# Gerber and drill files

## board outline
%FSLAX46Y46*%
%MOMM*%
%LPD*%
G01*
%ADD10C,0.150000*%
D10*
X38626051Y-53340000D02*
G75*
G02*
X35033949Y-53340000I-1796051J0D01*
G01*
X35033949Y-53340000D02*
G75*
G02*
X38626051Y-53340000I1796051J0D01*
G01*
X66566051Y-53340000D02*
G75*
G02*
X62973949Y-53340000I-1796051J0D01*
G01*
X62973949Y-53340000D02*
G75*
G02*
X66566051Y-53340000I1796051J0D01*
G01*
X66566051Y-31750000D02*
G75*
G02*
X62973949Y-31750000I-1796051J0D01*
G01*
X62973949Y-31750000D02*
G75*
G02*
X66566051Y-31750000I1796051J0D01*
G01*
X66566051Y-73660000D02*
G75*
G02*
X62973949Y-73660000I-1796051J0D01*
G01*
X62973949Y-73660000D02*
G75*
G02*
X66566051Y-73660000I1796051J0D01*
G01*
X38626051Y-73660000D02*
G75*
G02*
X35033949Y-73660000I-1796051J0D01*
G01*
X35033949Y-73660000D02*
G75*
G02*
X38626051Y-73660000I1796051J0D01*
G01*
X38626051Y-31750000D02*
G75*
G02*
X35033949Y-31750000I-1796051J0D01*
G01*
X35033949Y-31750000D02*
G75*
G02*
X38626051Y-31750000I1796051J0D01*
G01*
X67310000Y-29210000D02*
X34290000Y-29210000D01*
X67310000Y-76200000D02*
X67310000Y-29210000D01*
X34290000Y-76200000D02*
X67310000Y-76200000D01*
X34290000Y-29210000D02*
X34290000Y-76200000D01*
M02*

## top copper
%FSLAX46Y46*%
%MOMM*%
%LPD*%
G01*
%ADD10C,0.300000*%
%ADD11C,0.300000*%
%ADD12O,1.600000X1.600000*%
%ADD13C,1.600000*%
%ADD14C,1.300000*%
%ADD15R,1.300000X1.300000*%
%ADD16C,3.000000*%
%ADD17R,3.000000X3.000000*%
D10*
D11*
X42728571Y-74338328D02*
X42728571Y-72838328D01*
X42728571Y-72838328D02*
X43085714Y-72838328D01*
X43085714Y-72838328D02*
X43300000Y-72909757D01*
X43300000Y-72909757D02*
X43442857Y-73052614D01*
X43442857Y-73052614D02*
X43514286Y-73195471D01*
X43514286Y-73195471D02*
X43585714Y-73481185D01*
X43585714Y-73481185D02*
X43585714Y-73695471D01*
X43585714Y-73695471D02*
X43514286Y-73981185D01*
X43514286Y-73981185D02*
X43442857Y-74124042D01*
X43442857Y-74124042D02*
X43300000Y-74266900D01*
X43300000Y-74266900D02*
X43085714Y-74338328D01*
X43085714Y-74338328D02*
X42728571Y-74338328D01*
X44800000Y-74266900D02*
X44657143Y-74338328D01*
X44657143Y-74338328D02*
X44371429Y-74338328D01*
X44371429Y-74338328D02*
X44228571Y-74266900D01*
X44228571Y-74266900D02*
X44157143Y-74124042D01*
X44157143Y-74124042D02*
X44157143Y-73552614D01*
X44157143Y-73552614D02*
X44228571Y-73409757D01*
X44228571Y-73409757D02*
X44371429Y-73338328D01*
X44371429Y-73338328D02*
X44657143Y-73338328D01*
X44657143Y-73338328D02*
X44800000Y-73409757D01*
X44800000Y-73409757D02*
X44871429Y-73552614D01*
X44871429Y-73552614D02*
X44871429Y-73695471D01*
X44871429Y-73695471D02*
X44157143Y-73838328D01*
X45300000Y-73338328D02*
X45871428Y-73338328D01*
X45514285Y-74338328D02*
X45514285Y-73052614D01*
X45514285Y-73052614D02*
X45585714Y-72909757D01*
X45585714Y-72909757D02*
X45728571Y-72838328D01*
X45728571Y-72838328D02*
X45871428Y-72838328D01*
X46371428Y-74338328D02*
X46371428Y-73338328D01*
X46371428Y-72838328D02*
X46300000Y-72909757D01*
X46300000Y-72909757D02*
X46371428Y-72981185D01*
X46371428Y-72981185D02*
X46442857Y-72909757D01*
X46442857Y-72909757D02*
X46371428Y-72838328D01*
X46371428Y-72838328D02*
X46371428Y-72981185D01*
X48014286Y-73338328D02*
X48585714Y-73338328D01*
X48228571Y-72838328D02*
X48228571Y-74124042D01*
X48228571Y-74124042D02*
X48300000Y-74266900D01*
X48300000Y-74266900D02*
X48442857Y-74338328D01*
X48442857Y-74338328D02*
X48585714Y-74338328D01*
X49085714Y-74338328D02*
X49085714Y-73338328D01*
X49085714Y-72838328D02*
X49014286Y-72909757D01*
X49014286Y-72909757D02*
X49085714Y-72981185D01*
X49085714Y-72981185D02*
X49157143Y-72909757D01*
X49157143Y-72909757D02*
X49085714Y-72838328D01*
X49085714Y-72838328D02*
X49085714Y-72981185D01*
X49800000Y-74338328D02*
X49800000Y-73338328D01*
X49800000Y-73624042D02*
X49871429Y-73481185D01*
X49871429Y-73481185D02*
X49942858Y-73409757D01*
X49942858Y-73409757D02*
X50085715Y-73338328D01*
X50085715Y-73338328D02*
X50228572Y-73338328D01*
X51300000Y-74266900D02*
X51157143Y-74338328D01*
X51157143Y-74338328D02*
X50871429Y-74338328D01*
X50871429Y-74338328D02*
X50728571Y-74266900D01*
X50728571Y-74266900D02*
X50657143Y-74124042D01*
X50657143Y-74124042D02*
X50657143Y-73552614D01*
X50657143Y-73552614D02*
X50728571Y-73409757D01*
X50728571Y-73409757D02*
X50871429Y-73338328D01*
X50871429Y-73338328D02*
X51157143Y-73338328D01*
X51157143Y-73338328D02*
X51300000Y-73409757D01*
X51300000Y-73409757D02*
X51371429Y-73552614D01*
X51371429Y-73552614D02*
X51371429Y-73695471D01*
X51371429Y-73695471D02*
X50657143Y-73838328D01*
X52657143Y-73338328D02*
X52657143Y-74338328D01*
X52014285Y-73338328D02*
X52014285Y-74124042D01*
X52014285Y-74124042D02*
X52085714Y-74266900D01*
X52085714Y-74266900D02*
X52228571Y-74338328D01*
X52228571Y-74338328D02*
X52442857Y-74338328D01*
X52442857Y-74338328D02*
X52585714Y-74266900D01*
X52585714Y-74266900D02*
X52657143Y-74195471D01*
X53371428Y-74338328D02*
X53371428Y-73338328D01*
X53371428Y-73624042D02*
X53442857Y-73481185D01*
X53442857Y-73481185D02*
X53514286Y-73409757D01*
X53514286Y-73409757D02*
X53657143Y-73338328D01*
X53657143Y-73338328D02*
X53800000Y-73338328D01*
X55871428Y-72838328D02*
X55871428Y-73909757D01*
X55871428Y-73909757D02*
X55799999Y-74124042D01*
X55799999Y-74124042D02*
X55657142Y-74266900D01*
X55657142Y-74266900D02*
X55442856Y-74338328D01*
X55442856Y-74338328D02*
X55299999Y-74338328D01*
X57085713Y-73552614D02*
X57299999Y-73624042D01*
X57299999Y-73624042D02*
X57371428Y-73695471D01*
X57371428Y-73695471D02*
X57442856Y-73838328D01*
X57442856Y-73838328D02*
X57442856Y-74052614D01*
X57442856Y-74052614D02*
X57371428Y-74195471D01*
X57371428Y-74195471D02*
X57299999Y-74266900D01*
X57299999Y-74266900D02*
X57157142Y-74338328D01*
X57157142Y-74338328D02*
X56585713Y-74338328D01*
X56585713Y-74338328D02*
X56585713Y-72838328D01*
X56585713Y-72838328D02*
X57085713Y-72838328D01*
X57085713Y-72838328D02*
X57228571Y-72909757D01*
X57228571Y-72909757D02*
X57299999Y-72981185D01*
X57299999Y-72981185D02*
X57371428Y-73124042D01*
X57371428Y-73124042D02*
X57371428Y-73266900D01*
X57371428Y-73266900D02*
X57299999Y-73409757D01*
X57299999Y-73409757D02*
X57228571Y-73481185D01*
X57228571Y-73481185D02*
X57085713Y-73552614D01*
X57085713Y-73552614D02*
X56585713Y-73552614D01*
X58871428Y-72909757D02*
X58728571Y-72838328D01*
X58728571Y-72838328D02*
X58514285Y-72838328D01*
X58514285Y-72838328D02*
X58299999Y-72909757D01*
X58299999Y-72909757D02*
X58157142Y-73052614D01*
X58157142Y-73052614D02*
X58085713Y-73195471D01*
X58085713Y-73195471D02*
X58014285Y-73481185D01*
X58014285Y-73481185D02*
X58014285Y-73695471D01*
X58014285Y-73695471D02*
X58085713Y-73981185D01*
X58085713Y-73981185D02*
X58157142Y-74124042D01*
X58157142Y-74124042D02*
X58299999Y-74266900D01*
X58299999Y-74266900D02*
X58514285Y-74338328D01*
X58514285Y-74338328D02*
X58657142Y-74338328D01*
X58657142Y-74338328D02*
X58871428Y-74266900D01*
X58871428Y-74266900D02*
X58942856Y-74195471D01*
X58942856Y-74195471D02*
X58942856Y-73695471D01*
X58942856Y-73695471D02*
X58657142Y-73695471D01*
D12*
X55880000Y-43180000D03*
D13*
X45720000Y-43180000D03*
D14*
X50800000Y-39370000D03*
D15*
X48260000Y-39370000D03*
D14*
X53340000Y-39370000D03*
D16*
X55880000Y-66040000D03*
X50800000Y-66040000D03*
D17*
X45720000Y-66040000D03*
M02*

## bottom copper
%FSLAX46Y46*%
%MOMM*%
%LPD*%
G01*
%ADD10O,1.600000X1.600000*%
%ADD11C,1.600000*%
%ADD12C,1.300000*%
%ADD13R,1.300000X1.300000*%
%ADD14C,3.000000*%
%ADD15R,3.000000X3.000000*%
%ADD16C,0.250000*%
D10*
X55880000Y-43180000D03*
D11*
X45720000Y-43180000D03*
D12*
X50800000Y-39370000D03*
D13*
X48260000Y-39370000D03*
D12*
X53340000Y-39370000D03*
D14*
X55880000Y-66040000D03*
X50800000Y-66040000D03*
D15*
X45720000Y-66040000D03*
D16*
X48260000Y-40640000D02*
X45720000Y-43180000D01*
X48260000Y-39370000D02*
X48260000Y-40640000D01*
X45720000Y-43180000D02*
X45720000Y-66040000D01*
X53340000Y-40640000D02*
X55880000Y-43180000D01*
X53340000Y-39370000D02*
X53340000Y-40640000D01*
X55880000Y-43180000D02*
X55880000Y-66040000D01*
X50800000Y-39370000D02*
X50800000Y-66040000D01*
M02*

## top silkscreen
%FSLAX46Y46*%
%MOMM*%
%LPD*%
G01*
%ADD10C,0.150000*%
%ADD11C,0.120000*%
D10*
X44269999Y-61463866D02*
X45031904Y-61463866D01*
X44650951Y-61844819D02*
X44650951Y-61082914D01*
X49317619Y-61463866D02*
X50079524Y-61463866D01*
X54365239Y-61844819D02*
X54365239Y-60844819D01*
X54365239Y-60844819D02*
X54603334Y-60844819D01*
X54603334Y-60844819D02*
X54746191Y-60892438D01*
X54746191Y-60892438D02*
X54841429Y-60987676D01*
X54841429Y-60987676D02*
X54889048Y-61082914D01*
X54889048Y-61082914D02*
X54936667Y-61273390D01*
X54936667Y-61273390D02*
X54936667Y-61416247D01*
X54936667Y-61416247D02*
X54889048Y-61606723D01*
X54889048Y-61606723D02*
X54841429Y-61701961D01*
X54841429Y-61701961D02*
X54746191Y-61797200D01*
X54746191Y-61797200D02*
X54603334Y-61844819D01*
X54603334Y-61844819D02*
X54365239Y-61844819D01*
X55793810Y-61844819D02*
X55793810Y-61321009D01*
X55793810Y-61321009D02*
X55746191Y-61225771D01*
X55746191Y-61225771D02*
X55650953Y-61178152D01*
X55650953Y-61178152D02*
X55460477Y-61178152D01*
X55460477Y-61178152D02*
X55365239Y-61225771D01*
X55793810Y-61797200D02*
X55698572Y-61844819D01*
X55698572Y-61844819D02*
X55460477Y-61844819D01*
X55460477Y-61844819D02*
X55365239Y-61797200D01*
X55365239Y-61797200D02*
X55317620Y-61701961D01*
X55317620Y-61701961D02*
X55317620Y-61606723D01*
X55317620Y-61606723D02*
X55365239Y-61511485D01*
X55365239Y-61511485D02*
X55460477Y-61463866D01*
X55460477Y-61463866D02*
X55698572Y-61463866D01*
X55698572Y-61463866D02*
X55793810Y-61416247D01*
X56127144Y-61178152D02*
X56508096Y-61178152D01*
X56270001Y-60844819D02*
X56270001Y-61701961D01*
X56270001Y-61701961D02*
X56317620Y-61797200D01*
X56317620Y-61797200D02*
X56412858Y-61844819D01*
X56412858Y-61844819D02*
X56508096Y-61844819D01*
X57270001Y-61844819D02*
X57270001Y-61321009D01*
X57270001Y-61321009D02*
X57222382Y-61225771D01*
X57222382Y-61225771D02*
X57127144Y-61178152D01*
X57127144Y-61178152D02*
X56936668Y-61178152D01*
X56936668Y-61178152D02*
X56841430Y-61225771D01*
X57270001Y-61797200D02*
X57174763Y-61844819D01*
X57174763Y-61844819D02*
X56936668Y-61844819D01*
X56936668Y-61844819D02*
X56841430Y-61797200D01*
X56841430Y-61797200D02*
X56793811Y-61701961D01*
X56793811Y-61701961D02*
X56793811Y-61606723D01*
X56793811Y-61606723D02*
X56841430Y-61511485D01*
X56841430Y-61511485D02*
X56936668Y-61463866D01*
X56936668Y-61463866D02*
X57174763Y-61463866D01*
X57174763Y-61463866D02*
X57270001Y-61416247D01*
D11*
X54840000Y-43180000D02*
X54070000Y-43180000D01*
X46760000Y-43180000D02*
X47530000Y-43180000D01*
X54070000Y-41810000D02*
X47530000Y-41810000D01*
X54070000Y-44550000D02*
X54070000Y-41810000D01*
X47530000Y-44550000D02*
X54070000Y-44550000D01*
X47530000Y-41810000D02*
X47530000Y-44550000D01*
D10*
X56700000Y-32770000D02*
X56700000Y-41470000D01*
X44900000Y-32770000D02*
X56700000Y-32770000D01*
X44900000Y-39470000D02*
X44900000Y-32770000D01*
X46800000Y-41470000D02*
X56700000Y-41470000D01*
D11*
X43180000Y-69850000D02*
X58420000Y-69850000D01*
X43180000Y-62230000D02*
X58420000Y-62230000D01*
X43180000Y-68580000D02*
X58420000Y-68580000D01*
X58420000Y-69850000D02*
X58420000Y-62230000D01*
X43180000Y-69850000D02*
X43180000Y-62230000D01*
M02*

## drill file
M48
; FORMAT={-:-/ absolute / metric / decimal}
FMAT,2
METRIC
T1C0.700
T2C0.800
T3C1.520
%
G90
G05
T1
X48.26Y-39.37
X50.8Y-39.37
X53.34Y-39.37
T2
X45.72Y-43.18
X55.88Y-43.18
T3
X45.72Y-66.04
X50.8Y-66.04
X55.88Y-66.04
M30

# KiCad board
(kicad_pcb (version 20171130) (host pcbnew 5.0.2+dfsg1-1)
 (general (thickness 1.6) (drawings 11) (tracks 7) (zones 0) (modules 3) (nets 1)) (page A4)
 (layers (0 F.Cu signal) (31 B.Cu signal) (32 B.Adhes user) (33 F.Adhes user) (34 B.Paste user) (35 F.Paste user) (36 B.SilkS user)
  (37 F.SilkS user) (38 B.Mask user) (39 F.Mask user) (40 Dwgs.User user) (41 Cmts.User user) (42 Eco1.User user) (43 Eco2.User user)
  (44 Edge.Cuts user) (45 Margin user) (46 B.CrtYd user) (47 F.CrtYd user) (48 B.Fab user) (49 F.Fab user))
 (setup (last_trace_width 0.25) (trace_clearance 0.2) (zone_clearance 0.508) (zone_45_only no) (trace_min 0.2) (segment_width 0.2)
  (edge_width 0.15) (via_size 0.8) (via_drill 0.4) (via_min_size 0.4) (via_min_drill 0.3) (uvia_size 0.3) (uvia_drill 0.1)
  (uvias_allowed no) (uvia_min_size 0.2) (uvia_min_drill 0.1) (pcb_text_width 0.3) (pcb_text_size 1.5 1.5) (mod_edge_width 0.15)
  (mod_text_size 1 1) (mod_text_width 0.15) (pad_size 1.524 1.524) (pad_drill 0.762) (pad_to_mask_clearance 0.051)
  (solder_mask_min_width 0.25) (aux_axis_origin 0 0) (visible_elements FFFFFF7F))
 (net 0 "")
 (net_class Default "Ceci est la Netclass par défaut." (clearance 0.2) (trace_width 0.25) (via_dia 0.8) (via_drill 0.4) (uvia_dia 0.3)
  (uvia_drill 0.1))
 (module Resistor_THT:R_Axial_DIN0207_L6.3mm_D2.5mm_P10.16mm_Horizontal (layer F.Cu) (at 45.72 43.18)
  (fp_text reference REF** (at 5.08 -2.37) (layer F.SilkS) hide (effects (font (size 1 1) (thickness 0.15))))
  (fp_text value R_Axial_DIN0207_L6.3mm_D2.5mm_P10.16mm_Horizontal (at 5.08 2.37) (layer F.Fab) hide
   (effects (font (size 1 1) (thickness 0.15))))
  (fp_line (start 9.12 0) (end 8.35 0) (layer F.SilkS) (width 0.12))
  (fp_line (start 1.04 0) (end 1.81 0) (layer F.SilkS) (width 0.12))
  (fp_line (start 8.35 -1.37) (end 1.81 -1.37) (layer F.SilkS) (width 0.12))
  (fp_line (start 8.35 1.37) (end 8.35 -1.37) (layer F.SilkS) (width 0.12))
  (fp_line (start 1.81 1.37) (end 8.35 1.37) (layer F.SilkS) (width 0.12))
  (fp_line (start 1.81 -1.37) (end 1.81 1.37) (layer F.SilkS) (width 0.12))
  (pad 2 thru_hole oval (at 10.16 0) (size 1.6 1.6) (drill 0.8) (layers *.Cu *.Mask))
  (pad 1 thru_hole circle (at 0 0) (size 1.6 1.6) (drill 0.8) (layers *.Cu *.Mask)))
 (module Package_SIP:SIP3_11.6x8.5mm (layer F.Cu) (at 48.26 39.37)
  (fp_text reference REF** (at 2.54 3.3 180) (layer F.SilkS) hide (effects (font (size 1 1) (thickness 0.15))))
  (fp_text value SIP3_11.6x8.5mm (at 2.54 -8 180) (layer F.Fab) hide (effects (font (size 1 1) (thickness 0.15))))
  (fp_line (start 8.44 -6.6) (end 8.44 2.1) (layer F.SilkS) (width 0.15))
  (fp_line (start -3.36 -6.6) (end 8.44 -6.6) (layer F.SilkS) (width 0.15))
  (fp_line (start -3.36 0.1) (end -3.36 -6.6) (layer F.SilkS) (width 0.15))
  (fp_line (start -1.46 2.1) (end 8.44 2.1) (layer F.SilkS) (width 0.15))
  (pad 2 thru_hole circle (at 2.54 0 180) (size 1.3 1.3) (drill 0.7) (layers *.Cu *.Mask))
  (pad 1 thru_hole rect (at 0 0 270) (size 1.3 1.3) (drill 0.7) (layers *.Cu *.Mask))
  (pad 3 thru_hole circle (at 5.08 0 270) (size 1.3 1.3) (drill 0.7) (layers *.Cu *.Mask)))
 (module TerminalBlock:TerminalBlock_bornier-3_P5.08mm (layer F.Cu) (at 45.72 66.04)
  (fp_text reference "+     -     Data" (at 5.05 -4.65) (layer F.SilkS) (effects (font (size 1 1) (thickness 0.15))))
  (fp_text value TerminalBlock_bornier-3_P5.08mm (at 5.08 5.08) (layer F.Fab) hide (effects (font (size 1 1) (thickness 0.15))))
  (fp_line (start -2.54 3.81) (end 12.7 3.81) (layer F.SilkS) (width 0.12))
  (fp_line (start -2.54 -3.81) (end 12.7 -3.81) (layer F.SilkS) (width 0.12))
  (fp_line (start -2.54 2.54) (end 12.7 2.54) (layer F.SilkS) (width 0.12))
  (fp_line (start 12.7 3.81) (end 12.7 -3.81) (layer F.SilkS) (width 0.12))
  (fp_line (start -2.54 3.81) (end -2.54 -3.81) (layer F.SilkS) (width 0.12))
  (pad 3 thru_hole circle (at 10.16 0) (size 3 3) (drill 1.52) (layers *.Cu *.Mask))
  (pad 2 thru_hole circle (at 5.08 0) (size 3 3) (drill 1.52) (layers *.Cu *.Mask))
  (pad 1 thru_hole rect (at 0 0) (size 3 3) (drill 1.52) (layers *.Cu *.Mask)))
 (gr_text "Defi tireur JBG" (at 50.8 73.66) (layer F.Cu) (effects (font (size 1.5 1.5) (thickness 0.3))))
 (gr_circle (center 36.83 53.34) (end 38.1 54.61) (layer Edge.Cuts) (width 0.15))
 (gr_circle (center 64.77 53.34) (end 66.04 54.61) (layer Edge.Cuts) (width 0.15))
 (gr_circle (center 64.77 31.75) (end 66.04 33.02) (layer Edge.Cuts) (width 0.15))
 (gr_circle (center 64.77 73.66) (end 66.04 74.93) (layer Edge.Cuts) (width 0.15))
 (gr_circle (center 36.83 73.66) (end 38.1 74.93) (layer Edge.Cuts) (width 0.15))
 (gr_circle (center 36.83 31.75) (end 38.1 33.02) (layer Edge.Cuts) (width 0.15))
 (gr_line (start 67.31 29.21) (end 34.29 29.21) (layer Edge.Cuts) (width 0.15))
 (gr_line (start 67.31 76.2) (end 67.31 29.21) (layer Edge.Cuts) (width 0.15))
 (gr_line (start 34.29 76.2) (end 67.31 76.2) (layer Edge.Cuts) (width 0.15))
 (gr_line (start 34.29 29.21) (end 34.29 76.2) (layer Edge.Cuts) (width 0.15))
 (segment (start 48.26 40.64) (end 45.72 43.18) (width 0.25) (layer B.Cu) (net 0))
 (segment (start 48.26 39.37) (end 48.26 40.64) (width 0.25) (layer B.Cu) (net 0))
 (segment (start 45.72 43.18) (end 45.72 66.04) (width 0.25) (layer B.Cu) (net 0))
 (segment (start 53.34 40.64) (end 55.88 43.18) (width 0.25) (layer B.Cu) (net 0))
 (segment (start 53.34 39.37) (end 53.34 40.64) (width 0.25) (layer B.Cu) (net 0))
 (segment (start 55.88 43.18) (end 55.88 66.04) (width 0.25) (layer B.Cu) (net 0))
 (segment (start 50.8 39.37) (end 50.8 66.04) (width 0.25) (layer B.Cu) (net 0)))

